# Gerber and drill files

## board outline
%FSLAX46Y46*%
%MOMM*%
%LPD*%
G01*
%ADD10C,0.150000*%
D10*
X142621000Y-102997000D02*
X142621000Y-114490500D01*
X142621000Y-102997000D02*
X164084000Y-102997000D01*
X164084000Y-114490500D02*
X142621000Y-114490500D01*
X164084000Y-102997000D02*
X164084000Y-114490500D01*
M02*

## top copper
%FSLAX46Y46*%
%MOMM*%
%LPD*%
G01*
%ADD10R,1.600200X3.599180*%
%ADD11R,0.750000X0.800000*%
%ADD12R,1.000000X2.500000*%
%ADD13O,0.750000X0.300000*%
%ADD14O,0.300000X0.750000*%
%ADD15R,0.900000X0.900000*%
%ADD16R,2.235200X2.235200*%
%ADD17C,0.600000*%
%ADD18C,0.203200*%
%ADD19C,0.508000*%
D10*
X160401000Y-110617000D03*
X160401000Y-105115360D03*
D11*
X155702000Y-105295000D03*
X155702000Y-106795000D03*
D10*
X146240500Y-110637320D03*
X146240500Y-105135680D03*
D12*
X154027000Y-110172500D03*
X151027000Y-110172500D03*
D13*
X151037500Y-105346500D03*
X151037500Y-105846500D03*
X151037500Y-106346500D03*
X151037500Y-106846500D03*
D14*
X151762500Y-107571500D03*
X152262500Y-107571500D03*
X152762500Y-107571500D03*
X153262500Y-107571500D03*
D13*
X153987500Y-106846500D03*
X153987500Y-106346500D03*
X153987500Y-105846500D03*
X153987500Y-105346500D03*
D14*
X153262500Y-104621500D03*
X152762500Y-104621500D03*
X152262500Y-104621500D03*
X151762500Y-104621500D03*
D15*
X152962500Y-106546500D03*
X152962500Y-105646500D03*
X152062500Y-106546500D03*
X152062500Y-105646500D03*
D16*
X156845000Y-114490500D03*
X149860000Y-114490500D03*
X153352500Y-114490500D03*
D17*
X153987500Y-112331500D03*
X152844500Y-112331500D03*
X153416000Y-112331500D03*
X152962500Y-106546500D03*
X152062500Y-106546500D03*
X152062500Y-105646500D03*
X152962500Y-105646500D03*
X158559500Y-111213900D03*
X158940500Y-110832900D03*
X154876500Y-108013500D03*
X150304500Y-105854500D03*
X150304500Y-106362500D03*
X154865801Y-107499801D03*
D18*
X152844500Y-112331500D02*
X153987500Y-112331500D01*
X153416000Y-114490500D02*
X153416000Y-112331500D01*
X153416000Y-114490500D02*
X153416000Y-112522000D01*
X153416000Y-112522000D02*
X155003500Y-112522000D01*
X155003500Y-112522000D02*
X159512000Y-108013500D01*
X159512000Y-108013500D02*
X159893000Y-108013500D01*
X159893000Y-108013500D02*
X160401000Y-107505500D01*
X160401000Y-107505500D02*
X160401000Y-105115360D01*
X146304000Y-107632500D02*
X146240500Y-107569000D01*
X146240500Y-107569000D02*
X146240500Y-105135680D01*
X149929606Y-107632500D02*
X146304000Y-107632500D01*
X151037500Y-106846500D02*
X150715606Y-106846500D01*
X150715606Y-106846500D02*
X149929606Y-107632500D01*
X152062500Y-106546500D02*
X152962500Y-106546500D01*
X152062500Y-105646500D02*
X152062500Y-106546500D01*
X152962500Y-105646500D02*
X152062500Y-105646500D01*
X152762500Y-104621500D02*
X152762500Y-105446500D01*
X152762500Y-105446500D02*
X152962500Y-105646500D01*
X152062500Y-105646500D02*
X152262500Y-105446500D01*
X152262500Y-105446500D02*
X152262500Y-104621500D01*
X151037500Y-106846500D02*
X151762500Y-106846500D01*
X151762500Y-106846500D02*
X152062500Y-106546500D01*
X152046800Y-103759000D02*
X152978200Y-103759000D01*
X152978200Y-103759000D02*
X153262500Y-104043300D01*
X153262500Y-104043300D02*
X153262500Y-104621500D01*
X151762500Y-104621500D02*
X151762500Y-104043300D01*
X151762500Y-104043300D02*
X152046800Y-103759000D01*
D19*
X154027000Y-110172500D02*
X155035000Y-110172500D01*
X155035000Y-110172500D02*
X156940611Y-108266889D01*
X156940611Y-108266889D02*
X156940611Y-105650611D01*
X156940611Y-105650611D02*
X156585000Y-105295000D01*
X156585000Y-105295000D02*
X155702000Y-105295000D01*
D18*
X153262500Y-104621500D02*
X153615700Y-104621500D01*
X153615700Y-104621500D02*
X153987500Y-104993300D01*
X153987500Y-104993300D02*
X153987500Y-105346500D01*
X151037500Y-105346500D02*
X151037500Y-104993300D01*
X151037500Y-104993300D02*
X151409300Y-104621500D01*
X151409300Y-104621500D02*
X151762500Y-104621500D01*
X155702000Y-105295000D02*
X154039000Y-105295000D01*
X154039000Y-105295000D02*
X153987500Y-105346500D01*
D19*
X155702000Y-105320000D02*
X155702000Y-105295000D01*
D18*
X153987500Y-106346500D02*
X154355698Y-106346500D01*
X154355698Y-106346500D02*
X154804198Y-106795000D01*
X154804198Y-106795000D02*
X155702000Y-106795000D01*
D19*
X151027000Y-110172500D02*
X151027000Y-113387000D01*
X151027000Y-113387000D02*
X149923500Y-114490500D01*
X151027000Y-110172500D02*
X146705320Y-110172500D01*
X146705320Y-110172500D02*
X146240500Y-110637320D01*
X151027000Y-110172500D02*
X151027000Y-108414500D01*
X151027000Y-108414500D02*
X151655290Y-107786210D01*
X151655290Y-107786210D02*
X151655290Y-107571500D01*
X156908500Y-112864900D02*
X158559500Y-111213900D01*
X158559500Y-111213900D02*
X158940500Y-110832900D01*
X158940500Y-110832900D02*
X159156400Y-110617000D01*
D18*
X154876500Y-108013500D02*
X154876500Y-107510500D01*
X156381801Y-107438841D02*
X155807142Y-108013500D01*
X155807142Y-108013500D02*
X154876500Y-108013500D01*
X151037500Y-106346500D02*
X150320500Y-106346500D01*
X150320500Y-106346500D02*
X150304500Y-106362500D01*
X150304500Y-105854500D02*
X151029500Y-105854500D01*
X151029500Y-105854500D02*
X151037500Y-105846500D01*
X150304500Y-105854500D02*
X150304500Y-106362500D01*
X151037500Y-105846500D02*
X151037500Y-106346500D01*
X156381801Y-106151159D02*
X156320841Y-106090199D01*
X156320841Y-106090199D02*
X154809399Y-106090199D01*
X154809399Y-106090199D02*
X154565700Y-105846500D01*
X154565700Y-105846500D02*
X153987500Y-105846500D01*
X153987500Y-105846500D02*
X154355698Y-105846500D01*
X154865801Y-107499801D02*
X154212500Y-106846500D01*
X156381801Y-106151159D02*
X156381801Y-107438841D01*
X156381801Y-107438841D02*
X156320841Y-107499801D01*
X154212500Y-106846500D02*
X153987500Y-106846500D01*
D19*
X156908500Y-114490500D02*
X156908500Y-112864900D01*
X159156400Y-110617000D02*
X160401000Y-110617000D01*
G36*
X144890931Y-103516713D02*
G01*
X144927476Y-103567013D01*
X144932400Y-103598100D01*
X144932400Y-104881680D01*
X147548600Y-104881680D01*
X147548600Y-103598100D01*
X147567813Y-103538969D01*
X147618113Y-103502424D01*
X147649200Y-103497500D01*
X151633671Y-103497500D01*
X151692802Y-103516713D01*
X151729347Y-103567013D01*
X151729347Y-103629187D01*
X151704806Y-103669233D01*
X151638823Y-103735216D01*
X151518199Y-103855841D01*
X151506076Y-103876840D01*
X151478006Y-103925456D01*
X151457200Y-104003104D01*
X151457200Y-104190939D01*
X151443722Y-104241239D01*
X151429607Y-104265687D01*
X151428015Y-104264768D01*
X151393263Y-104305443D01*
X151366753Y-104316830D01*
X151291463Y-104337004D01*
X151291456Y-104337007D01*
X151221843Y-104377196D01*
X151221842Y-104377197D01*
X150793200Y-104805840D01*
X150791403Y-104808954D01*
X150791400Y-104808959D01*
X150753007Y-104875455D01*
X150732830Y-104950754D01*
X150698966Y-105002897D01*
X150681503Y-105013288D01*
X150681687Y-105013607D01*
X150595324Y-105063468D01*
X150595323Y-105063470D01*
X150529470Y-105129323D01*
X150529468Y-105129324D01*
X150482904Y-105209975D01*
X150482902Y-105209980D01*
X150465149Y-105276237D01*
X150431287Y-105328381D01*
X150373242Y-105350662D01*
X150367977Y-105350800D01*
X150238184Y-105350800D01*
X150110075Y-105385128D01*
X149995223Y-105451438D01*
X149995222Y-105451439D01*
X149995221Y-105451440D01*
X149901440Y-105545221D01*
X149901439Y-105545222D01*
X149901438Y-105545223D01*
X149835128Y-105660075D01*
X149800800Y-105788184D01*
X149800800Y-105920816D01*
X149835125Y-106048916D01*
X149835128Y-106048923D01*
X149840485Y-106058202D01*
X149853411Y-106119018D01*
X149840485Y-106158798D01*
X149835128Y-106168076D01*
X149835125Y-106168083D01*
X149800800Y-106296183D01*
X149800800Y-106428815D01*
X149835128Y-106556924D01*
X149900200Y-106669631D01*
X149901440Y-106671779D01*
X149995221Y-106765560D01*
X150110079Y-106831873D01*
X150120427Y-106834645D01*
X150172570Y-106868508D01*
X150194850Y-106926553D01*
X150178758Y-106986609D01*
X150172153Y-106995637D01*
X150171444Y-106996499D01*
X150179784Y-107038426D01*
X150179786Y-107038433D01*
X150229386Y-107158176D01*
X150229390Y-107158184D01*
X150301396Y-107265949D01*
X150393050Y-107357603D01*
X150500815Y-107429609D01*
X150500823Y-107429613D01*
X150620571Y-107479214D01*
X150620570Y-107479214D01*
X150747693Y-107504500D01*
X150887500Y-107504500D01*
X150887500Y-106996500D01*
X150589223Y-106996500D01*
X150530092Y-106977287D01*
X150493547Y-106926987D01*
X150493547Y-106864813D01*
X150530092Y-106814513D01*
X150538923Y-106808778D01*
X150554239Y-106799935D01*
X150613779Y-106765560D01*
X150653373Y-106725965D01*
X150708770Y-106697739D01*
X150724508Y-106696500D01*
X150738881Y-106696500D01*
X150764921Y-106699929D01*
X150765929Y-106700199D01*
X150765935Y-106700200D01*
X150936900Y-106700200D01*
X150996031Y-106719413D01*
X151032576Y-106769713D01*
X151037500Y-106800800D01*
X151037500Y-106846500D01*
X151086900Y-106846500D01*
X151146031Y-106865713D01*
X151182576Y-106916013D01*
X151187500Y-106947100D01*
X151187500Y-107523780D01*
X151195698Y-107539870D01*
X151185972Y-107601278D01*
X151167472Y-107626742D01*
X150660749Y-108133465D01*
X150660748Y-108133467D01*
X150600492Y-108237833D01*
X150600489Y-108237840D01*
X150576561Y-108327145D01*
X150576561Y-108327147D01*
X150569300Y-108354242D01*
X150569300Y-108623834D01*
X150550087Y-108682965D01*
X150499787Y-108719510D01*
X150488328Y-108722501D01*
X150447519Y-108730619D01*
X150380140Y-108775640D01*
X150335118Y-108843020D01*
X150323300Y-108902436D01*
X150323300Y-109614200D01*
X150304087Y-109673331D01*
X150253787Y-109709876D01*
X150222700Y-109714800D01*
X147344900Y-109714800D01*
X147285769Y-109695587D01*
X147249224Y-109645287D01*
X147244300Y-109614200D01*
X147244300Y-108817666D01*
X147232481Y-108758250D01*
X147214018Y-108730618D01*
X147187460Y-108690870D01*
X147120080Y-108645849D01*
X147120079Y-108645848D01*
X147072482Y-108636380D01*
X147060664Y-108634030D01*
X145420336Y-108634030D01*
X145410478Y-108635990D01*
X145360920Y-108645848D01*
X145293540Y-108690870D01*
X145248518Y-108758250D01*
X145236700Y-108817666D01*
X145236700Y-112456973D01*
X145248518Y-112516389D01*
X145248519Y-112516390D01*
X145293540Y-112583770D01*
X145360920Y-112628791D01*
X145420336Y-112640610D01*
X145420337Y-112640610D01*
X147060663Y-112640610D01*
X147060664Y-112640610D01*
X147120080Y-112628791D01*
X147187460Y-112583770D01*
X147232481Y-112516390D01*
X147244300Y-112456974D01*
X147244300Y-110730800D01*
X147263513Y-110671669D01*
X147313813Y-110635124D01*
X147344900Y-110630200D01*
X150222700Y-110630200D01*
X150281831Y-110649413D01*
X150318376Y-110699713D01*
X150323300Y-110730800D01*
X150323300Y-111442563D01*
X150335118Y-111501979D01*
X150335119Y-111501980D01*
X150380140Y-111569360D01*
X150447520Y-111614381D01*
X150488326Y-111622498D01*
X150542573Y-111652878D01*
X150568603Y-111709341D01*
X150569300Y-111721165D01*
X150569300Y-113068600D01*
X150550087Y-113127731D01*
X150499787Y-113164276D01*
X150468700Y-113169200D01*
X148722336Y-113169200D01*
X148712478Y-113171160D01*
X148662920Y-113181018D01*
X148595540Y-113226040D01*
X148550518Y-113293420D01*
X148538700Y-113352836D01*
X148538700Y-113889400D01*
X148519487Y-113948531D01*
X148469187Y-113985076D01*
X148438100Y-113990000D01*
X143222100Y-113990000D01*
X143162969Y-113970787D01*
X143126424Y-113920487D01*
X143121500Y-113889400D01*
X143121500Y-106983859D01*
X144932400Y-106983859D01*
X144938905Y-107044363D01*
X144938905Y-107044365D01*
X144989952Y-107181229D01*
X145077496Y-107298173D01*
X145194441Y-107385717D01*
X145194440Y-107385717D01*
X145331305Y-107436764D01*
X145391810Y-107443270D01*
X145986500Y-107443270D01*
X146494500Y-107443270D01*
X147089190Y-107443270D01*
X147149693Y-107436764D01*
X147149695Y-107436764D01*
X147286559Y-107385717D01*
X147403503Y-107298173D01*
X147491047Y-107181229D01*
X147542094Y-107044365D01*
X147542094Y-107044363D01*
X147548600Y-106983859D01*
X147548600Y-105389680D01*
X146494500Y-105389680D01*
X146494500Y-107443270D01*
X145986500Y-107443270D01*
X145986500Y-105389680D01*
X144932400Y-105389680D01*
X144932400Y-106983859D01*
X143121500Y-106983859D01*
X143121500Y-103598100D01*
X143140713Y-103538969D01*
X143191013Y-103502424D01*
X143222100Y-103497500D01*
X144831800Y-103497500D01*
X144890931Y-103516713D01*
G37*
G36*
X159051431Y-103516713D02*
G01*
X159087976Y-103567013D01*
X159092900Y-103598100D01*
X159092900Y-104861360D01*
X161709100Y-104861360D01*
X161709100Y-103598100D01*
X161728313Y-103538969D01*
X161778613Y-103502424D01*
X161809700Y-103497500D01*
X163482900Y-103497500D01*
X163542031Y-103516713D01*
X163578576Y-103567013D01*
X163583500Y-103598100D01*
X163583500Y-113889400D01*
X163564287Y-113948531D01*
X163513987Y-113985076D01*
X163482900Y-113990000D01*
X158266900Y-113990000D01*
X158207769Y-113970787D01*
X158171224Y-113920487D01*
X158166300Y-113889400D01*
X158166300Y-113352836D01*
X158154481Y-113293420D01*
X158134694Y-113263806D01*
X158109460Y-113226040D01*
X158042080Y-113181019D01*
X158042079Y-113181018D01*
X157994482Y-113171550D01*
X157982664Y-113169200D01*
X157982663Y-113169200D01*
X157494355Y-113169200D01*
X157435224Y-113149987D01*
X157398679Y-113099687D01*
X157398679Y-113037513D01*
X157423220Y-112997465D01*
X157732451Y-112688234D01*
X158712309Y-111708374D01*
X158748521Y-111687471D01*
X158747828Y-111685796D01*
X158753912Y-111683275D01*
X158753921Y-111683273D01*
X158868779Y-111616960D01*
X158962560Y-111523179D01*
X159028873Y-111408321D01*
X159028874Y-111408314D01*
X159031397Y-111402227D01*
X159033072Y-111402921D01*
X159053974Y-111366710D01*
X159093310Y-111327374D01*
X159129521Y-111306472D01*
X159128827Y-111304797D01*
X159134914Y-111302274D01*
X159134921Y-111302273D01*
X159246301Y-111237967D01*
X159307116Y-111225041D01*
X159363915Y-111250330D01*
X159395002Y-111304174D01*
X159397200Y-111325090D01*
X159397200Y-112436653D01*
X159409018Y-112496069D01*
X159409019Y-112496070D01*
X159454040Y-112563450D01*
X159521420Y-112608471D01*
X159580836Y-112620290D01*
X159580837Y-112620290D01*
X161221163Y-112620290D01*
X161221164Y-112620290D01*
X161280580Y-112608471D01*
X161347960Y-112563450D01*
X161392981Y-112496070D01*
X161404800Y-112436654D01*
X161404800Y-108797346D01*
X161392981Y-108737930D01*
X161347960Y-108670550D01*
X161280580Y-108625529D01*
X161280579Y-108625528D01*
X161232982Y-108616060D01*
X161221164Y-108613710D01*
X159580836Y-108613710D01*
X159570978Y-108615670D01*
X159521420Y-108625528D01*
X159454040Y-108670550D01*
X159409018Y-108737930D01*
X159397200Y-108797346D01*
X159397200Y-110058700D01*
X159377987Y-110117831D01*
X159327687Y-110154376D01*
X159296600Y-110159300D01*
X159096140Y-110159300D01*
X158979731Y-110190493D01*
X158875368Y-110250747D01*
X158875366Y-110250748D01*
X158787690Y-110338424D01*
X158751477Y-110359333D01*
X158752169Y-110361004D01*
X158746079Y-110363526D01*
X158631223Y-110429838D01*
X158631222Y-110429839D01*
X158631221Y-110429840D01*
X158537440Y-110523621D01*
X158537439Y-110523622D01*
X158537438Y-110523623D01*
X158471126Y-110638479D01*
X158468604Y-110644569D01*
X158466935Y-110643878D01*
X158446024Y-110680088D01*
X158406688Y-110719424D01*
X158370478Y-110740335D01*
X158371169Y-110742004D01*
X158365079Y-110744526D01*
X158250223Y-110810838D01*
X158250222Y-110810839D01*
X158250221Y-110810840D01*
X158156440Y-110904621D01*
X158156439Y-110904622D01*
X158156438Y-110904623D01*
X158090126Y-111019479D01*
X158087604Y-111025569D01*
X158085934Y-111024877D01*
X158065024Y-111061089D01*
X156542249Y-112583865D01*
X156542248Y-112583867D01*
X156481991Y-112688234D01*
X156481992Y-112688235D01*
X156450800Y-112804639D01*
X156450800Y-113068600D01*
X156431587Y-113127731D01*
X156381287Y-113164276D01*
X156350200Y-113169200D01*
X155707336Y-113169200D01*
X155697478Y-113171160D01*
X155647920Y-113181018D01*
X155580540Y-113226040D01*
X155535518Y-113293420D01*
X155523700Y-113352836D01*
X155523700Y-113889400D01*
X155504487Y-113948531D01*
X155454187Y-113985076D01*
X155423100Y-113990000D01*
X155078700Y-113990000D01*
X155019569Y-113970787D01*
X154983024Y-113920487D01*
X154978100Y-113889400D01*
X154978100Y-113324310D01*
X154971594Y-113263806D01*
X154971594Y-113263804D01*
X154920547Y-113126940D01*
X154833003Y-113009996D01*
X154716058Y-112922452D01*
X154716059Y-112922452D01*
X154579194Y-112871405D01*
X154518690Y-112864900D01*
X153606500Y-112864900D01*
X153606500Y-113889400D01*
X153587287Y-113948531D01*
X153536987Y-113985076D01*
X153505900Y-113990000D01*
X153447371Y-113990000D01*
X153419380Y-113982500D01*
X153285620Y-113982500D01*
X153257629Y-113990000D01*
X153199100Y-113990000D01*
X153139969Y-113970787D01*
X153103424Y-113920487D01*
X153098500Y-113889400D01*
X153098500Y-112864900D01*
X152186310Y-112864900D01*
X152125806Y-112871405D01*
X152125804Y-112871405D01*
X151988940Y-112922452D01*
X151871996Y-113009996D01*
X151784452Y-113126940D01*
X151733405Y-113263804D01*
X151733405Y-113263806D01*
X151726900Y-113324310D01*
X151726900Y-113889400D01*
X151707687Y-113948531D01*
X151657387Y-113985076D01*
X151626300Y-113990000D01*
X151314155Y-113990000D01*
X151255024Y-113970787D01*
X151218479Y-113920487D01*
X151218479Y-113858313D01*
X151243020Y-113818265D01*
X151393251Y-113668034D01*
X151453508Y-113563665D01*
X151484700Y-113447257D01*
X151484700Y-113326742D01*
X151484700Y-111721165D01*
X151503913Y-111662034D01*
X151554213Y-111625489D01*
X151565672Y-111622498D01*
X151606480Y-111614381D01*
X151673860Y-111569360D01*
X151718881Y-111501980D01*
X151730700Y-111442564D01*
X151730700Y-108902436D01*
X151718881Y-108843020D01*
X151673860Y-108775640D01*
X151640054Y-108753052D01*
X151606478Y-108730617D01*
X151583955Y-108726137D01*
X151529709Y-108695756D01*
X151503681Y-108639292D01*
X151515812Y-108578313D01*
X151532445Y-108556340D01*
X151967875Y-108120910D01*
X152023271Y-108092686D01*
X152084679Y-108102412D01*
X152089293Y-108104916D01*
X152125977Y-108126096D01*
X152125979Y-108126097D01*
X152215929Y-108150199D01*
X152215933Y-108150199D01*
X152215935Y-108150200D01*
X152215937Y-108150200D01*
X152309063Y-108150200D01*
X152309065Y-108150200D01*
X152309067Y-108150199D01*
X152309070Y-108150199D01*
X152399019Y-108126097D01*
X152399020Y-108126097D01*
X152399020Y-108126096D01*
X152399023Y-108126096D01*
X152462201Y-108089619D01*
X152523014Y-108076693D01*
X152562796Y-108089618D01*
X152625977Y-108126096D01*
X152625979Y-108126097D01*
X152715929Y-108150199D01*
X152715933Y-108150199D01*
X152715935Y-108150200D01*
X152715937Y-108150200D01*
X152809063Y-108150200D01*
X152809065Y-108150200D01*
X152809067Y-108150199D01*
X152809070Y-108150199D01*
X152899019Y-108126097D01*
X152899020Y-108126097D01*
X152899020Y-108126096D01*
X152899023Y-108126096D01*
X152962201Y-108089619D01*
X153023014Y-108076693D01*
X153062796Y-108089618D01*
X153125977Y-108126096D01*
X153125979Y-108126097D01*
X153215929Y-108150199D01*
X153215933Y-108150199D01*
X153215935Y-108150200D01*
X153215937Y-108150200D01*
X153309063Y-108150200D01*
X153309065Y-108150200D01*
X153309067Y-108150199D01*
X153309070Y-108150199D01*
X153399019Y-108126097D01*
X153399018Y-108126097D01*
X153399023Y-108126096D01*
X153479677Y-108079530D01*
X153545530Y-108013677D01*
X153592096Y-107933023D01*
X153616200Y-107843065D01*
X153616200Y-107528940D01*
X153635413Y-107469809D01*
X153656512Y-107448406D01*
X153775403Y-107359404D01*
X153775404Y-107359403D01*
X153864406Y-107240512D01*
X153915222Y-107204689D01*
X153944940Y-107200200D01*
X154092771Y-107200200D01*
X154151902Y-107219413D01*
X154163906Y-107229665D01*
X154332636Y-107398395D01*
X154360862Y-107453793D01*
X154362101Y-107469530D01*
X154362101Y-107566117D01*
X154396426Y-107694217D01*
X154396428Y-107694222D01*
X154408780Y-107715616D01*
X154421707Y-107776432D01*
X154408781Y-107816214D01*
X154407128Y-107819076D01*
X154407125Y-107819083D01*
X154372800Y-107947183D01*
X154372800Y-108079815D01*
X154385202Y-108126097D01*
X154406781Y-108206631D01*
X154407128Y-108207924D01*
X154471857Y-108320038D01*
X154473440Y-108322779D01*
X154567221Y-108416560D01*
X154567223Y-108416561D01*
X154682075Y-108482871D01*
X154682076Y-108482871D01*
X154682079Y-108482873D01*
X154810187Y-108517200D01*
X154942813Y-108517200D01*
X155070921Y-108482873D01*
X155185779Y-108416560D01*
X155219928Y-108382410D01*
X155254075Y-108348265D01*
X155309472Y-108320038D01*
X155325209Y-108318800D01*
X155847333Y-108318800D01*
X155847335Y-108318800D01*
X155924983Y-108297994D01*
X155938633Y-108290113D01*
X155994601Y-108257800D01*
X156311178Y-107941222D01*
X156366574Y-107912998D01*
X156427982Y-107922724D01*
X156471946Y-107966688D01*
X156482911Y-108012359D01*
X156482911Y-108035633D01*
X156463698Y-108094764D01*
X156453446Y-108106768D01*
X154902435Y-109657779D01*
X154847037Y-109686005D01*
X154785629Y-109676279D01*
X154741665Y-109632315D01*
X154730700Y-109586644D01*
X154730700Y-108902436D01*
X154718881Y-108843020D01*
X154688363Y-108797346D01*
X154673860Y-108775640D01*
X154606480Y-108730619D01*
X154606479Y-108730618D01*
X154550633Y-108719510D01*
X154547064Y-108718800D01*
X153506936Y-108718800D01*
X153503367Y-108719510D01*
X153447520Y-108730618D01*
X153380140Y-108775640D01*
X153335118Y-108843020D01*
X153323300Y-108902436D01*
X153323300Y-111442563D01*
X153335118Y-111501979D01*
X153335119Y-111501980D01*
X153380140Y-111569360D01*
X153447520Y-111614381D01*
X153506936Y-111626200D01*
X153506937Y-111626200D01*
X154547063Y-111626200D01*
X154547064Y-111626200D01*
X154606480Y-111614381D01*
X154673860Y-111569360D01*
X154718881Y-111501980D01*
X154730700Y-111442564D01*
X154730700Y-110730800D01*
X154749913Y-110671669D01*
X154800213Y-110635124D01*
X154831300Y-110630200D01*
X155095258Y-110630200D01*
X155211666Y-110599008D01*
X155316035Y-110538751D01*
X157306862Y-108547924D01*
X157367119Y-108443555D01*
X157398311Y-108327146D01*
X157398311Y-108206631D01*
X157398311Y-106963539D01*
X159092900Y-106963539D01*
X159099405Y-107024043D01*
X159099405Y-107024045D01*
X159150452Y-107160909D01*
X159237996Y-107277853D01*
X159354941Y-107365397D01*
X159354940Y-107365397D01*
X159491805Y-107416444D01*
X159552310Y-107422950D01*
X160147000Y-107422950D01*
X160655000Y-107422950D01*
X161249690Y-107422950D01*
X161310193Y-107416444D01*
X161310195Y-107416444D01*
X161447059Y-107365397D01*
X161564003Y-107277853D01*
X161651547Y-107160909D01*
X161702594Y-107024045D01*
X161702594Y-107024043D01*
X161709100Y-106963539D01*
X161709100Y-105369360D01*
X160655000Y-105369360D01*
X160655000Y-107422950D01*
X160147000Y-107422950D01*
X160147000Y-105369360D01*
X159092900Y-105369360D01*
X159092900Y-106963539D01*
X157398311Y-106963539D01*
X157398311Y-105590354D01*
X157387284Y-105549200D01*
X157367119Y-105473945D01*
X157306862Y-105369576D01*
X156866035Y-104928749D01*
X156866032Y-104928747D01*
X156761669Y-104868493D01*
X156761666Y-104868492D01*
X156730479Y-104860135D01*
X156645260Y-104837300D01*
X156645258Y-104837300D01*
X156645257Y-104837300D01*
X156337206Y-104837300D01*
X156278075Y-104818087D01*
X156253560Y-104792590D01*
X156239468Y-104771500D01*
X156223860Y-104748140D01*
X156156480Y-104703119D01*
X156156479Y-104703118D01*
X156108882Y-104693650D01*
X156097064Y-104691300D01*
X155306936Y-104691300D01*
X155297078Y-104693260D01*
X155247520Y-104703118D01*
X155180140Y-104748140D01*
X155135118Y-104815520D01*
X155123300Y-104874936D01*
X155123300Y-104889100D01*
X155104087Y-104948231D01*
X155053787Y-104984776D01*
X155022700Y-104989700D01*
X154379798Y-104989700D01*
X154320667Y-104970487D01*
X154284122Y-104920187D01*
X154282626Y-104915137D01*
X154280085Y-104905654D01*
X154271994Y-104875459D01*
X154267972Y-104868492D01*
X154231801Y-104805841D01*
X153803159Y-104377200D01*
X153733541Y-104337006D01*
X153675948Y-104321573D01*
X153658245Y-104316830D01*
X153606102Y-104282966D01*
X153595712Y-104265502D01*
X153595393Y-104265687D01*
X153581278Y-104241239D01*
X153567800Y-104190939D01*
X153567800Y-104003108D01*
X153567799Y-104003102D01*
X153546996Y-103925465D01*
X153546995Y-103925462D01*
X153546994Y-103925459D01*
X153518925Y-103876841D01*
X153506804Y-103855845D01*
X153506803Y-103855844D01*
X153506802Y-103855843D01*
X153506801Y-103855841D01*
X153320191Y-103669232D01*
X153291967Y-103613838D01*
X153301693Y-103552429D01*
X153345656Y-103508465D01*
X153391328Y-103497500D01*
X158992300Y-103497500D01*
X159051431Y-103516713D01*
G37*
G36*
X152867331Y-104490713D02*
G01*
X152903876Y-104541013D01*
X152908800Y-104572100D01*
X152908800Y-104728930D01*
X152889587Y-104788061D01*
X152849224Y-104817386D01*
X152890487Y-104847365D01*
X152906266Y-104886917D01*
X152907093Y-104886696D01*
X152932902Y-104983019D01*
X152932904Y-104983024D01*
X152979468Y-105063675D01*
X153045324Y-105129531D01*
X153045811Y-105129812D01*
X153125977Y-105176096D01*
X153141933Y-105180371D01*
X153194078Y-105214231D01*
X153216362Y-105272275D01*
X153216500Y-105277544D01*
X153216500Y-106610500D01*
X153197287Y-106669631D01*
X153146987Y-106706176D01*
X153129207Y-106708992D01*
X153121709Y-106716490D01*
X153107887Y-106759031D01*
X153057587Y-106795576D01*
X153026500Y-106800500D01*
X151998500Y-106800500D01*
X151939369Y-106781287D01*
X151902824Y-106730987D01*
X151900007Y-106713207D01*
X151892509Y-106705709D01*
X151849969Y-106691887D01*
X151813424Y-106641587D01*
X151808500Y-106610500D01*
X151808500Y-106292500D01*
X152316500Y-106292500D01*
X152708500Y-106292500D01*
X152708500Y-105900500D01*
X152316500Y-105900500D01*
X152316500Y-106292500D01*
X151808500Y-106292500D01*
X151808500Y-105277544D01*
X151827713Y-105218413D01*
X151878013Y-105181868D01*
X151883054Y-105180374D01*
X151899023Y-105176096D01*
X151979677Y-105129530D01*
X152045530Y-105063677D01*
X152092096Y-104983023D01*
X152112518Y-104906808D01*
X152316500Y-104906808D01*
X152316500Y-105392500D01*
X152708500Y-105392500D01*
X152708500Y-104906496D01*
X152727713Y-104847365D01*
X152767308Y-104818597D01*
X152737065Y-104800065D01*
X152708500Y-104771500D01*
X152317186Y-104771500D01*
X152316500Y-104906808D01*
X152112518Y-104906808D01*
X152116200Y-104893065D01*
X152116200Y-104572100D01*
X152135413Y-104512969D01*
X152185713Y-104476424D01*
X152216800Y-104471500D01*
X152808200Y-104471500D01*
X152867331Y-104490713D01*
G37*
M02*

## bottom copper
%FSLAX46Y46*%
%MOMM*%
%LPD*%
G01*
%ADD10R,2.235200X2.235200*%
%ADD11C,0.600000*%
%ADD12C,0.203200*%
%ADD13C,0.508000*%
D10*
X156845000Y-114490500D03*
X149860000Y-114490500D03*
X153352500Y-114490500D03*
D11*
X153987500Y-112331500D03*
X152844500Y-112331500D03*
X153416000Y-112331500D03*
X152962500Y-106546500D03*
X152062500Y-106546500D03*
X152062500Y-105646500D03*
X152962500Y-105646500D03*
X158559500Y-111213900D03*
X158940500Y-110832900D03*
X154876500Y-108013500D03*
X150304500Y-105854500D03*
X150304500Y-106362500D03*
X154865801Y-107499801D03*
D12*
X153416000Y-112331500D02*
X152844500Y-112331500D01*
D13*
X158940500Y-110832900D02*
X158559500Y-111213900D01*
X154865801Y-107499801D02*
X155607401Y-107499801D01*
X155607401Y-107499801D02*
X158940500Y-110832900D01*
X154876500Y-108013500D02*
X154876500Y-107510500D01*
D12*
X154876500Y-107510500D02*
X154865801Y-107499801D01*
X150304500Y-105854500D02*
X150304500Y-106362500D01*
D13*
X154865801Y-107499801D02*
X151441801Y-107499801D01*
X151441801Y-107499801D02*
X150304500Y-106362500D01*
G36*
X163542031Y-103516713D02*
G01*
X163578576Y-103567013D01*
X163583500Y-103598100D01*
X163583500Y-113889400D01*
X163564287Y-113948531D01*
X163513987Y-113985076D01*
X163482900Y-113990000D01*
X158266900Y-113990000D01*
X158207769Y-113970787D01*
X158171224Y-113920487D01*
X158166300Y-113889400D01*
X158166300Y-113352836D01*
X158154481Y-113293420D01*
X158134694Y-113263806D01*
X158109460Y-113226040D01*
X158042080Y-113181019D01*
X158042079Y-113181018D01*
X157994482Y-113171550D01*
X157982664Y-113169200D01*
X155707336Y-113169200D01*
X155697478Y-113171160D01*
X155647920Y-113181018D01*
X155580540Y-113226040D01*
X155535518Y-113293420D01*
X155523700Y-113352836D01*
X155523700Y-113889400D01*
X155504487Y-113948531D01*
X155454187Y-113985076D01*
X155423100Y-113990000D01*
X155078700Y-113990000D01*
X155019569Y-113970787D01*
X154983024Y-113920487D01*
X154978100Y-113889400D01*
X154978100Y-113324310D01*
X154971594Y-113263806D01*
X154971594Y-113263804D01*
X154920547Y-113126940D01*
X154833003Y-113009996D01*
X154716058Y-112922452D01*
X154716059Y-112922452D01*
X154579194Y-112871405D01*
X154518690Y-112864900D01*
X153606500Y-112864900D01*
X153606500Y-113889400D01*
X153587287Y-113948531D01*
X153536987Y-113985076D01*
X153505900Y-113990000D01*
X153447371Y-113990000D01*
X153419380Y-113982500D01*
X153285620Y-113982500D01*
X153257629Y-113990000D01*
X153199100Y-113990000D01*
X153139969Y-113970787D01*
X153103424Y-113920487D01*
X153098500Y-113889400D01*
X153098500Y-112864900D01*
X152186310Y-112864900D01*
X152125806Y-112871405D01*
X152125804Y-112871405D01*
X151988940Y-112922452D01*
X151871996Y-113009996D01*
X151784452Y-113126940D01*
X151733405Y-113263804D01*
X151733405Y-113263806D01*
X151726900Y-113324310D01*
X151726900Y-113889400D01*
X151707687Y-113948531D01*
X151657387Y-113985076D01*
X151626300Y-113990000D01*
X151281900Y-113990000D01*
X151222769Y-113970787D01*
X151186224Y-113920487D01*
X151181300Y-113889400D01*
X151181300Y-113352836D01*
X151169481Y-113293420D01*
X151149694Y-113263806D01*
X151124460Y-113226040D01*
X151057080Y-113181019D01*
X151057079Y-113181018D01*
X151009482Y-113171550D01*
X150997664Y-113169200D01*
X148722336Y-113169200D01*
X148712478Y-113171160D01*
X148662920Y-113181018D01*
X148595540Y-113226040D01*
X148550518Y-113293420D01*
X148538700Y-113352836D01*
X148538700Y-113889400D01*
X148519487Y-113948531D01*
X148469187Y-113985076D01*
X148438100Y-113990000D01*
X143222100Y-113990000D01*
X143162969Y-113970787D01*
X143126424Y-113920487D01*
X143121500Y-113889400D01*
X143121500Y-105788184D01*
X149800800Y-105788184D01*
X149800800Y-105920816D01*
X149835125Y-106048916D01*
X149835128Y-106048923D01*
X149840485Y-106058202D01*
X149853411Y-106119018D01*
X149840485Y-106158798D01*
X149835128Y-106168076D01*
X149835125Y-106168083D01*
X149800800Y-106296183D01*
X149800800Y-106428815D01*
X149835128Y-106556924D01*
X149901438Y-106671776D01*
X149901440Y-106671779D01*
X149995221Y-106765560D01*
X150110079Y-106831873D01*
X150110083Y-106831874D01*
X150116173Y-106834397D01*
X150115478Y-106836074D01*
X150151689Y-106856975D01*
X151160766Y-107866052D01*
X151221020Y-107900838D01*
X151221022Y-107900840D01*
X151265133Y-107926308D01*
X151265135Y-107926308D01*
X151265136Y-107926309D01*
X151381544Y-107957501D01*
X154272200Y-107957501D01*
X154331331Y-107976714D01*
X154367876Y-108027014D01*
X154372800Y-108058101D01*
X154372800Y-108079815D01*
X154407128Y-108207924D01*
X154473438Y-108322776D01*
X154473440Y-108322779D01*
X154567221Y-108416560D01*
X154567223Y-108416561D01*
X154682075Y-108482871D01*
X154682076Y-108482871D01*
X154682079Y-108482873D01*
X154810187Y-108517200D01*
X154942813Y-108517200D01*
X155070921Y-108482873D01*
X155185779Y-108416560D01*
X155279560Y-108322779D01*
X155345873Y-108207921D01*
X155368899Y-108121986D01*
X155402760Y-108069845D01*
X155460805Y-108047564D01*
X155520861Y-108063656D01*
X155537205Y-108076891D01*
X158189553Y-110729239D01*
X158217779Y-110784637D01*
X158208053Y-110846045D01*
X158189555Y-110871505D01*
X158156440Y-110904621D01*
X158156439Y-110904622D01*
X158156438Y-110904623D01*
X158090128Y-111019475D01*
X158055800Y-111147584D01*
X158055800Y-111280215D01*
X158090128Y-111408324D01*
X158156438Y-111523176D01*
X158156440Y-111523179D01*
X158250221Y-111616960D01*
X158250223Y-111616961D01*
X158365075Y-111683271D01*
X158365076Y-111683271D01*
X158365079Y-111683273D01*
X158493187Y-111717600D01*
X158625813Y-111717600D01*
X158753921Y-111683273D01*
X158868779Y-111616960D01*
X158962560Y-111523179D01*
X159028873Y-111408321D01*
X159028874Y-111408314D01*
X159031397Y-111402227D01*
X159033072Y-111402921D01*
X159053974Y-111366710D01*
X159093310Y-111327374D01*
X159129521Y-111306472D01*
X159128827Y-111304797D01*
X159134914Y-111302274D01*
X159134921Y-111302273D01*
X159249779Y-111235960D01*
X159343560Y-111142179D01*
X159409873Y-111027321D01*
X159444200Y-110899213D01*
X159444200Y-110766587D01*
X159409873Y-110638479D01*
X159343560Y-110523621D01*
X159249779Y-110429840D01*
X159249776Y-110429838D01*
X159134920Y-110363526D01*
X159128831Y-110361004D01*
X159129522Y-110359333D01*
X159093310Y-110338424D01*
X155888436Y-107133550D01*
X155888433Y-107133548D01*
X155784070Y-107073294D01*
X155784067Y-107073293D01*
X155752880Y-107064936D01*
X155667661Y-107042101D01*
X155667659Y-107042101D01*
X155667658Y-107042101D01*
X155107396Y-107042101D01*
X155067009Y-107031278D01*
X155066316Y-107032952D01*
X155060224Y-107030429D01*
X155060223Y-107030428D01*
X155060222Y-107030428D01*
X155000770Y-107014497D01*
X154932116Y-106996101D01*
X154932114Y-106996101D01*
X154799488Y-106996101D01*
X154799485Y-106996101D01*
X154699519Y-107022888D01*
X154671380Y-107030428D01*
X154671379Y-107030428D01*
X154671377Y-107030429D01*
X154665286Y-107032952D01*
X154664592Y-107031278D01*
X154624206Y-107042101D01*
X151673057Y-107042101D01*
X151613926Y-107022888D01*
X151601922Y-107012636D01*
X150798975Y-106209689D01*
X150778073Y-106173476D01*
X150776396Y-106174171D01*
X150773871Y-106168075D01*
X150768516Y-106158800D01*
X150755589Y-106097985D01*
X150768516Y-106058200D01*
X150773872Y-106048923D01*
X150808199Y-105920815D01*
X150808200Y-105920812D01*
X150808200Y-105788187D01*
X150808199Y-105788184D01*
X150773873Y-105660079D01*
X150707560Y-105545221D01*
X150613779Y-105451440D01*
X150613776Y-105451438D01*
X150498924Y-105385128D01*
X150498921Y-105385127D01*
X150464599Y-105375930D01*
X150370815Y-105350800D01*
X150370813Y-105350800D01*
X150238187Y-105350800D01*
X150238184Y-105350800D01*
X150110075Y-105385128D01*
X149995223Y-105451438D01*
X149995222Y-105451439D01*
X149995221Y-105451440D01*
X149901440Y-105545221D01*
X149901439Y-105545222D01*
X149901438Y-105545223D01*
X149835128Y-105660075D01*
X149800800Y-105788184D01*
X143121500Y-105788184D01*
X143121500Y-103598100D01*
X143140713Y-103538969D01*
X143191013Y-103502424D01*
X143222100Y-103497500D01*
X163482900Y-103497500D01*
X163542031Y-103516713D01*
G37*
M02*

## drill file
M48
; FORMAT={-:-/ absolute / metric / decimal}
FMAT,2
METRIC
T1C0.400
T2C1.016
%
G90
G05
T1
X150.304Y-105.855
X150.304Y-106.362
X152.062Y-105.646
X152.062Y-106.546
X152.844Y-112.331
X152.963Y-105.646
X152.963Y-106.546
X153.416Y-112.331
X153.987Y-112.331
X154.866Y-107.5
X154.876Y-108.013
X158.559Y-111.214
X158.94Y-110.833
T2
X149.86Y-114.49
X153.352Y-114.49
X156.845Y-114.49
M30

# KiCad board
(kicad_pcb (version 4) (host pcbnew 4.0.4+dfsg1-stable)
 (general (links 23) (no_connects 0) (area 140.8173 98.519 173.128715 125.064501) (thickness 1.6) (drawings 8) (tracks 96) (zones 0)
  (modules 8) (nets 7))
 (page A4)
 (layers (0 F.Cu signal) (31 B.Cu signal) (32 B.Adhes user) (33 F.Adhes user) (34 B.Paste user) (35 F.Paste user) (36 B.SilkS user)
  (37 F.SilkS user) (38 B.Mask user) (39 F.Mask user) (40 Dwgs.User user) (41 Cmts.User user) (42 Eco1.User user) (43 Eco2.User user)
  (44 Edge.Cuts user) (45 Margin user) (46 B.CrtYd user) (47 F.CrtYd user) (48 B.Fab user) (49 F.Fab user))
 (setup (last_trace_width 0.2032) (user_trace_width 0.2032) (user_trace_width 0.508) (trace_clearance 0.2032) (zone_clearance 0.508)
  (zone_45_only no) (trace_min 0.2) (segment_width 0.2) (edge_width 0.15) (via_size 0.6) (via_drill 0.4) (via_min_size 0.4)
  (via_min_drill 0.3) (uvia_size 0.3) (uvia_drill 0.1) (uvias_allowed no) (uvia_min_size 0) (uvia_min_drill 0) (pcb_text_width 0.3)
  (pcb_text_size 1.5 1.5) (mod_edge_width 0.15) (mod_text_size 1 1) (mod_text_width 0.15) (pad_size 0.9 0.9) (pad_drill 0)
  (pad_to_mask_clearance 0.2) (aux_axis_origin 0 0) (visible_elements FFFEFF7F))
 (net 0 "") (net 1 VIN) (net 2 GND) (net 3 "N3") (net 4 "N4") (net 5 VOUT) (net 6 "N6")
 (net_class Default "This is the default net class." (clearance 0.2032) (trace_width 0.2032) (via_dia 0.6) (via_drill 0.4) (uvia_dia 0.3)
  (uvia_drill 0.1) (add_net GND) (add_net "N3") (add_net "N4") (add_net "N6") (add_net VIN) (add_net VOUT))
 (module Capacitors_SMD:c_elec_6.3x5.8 (layer F.Cu) (at 160.401 107.86618 270)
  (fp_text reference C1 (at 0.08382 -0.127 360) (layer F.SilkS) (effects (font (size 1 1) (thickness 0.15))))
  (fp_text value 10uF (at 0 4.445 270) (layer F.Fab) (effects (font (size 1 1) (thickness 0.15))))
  (pad 1 smd rect (at 2.75082 0 270) (size 3.59918 1.6002) (layers F.Cu F.Paste F.Mask) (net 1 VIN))
  (pad 2 smd rect (at -2.75082 0 270) (size 3.59918 1.6002) (layers F.Cu F.Paste F.Mask) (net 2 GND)))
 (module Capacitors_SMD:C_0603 (layer F.Cu) (at 155.702 106.045 270)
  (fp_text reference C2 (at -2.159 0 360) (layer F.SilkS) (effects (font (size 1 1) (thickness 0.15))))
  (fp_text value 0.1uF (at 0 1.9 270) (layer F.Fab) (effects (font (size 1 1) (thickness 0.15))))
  (pad 1 smd rect (at -0.75 0 270) (size 0.8 0.75) (layers F.Cu F.Paste F.Mask) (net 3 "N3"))
  (pad 2 smd rect (at 0.75 0 270) (size 0.8 0.75) (layers F.Cu F.Paste F.Mask) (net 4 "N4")))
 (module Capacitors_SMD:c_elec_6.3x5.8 (layer F.Cu) (at 146.2405 107.8865 270)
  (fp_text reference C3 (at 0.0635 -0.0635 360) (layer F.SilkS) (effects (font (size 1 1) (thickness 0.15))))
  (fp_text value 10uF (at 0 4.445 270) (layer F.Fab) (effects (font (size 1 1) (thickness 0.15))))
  (pad 1 smd rect (at 2.75082 0 270) (size 3.59918 1.6002) (layers F.Cu F.Paste F.Mask) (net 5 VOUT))
  (pad 2 smd rect (at -2.75082 0 270) (size 3.59918 1.6002) (layers F.Cu F.Paste F.Mask) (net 2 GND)))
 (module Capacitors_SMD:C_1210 (layer F.Cu) (at 152.527 110.1725 180)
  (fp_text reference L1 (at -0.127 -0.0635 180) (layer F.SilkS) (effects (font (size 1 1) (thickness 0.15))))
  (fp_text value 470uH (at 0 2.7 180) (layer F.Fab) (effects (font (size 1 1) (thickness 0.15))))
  (pad 1 smd rect (at -1.5 0 180) (size 1 2.5) (layers F.Cu F.Paste F.Mask) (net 3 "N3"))
  (pad 2 smd rect (at 1.5 0 180) (size 1 2.5) (layers F.Cu F.Paste F.Mask) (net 5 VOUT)))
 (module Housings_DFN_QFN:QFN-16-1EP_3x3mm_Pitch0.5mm (layer F.Cu) (at 152.5125 106.0965)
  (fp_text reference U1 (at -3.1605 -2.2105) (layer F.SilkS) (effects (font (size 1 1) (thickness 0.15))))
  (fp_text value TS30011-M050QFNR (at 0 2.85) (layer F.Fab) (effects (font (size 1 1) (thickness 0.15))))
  (pad 1 smd oval (at -1.475 -0.75) (size 0.75 0.3) (layers F.Cu F.Paste F.Mask) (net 3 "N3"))
  (pad 2 smd oval (at -1.475 -0.25) (size 0.75 0.3) (layers F.Cu F.Paste F.Mask) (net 1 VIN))
  (pad 3 smd oval (at -1.475 0.25) (size 0.75 0.3) (layers F.Cu F.Paste F.Mask) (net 1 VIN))
  (pad 4 smd oval (at -1.475 0.75) (size 0.75 0.3) (layers F.Cu F.Paste F.Mask) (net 2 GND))
  (pad 5 smd oval (at -0.75 1.475 90) (size 0.75 0.3) (layers F.Cu F.Paste F.Mask) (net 5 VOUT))
  (pad 6 smd oval (at -0.25 1.475 90) (size 0.75 0.3) (layers F.Cu F.Paste F.Mask))
  (pad 7 smd oval (at 0.25 1.475 90) (size 0.75 0.3) (layers F.Cu F.Paste F.Mask))
  (pad 8 smd oval (at 0.75 1.475 90) (size 0.75 0.3) (layers F.Cu F.Paste F.Mask) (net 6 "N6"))
  (pad 9 smd oval (at 1.475 0.75) (size 0.75 0.3) (layers F.Cu F.Paste F.Mask) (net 1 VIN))
  (pad 10 smd oval (at 1.475 0.25) (size 0.75 0.3) (layers F.Cu F.Paste F.Mask) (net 4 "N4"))
  (pad 11 smd oval (at 1.475 -0.25) (size 0.75 0.3) (layers F.Cu F.Paste F.Mask) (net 1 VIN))
  (pad 12 smd oval (at 1.475 -0.75) (size 0.75 0.3) (layers F.Cu F.Paste F.Mask) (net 3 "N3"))
  (pad 13 smd oval (at 0.75 -1.475 90) (size 0.75 0.3) (layers F.Cu F.Paste F.Mask) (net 3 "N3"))
  (pad 14 smd oval (at 0.25 -1.475 90) (size 0.75 0.3) (layers F.Cu F.Paste F.Mask) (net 2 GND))
  (pad 15 smd oval (at -0.25 -1.475 90) (size 0.75 0.3) (layers F.Cu F.Paste F.Mask) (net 2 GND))
  (pad 16 smd oval (at -0.75 -1.475 90) (size 0.75 0.3) (layers F.Cu F.Paste F.Mask) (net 3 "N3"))
  (pad 17 smd rect (at 0.45 0.45) (size 0.9 0.9) (layers F.Cu F.Paste F.Mask) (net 2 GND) (solder_paste_margin_ratio -0.2))
  (pad 17 smd rect (at 0.45 -0.45) (size 0.9 0.9) (layers F.Cu F.Paste F.Mask) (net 2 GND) (solder_paste_margin_ratio -0.2))
  (pad 17 smd rect (at -0.45 0.45) (size 0.9 0.9) (layers F.Cu F.Paste F.Mask) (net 2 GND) (solder_paste_margin_ratio -0.2))
  (pad 17 smd rect (at -0.45 -0.45) (size 0.9 0.9) (layers F.Cu F.Paste F.Mask) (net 2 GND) (solder_paste_margin_ratio -0.2)))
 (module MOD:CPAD (layer F.Cu) (at 156.845 114.4905)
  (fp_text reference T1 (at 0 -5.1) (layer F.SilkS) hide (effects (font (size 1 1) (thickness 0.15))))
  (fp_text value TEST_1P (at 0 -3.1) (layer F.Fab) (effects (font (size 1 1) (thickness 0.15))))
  (pad 1 thru_hole rect (at 0 0) (size 2.2352 2.2352) (drill 1.016) (layers *.Cu *.Mask F.SilkS) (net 1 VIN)))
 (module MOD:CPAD (layer F.Cu) (at 149.86 114.4905)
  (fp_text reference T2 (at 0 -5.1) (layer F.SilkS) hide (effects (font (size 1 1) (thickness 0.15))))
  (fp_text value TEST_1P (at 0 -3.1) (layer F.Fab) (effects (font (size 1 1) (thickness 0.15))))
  (pad 1 thru_hole rect (at 0 0) (size 2.2352 2.2352) (drill 1.016) (layers *.Cu *.Mask F.SilkS) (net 5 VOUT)))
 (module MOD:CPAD (layer F.Cu) (at 153.3525 114.4905)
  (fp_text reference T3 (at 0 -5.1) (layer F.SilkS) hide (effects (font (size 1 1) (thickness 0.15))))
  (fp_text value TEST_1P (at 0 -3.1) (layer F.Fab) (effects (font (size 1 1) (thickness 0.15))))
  (pad 1 thru_hole rect (at 0 0) (size 2.2352 2.2352) (drill 1.016) (layers *.Cu *.Mask F.SilkS) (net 2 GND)))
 (gr_line (start 142.621 102.997) (end 142.621 114.4905) (layer Edge.Cuts) (width 0.15))
 (gr_line (start 142.621 102.997) (end 164.084 102.997) (layer Edge.Cuts) (width 0.15))
 (gr_line (start 164.084 114.4905) (end 142.621 114.4905) (layer Edge.Cuts) (width 0.15))
 (gr_line (start 164.084 102.997) (end 164.084 114.4905) (layer Edge.Cuts) (width 0.15))
 (segment (start 152.8445 112.3315) (end 153.9875 112.3315) (width 0.2032) (layer F.Cu) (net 2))
 (via (at 153.9875 112.3315) (size 0.6) (drill 0.4) (layers F.Cu B.Cu) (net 2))
 (segment (start 153.416 112.3315) (end 152.8445 112.3315) (width 0.2032) (layer B.Cu) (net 2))
 (via (at 152.8445 112.3315) (size 0.6) (drill 0.4) (layers F.Cu B.Cu) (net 2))
 (segment (start 153.416 114.4905) (end 153.416 112.3315) (width 0.2032) (layer F.Cu) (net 2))
 (via (at 153.416 112.3315) (size 0.6) (drill 0.4) (layers F.Cu B.Cu) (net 2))
 (segment (start 153.416 114.4905) (end 153.416 112.522) (width 0.2032) (layer F.Cu) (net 2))
 (segment (start 153.416 112.522) (end 155.0035 112.522) (width 0.2032) (layer F.Cu) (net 2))
 (segment (start 155.0035 112.522) (end 159.512 108.0135) (width 0.2032) (layer F.Cu) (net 2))
 (segment (start 159.512 108.0135) (end 159.893 108.0135) (width 0.2032) (layer F.Cu) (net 2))
 (segment (start 159.893 108.0135) (end 160.401 107.5055) (width 0.2032) (layer F.Cu) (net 2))
 (segment (start 160.401 107.5055) (end 160.401 105.11536) (width 0.2032) (layer F.Cu) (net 2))
 (segment (start 146.304 107.6325) (end 146.2405 107.569) (width 0.2032) (layer F.Cu) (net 2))
 (segment (start 146.2405 107.569) (end 146.2405 105.13568) (width 0.2032) (layer F.Cu) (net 2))
 (segment (start 149.929606 107.6325) (end 146.304 107.6325) (width 0.2032) (layer F.Cu) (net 2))
 (segment (start 151.0375 106.8465) (end 150.715606 106.8465) (width 0.2032) (layer F.Cu) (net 2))
 (segment (start 150.715606 106.8465) (end 149.929606 107.6325) (width 0.2032) (layer F.Cu) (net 2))
 (segment (start 152.0625 106.5465) (end 152.9625 106.5465) (width 0.2032) (layer F.Cu) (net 2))
 (via (at 152.9625 106.5465) (size 0.6) (drill 0.4) (layers F.Cu B.Cu) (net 2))
 (segment (start 152.0625 105.6465) (end 152.0625 106.5465) (width 0.2032) (layer F.Cu) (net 2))
 (via (at 152.0625 106.5465) (size 0.6) (drill 0.4) (layers F.Cu B.Cu) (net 2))
 (segment (start 152.9625 105.6465) (end 152.0625 105.6465) (width 0.2032) (layer F.Cu) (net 2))
 (via (at 152.0625 105.6465) (size 0.6) (drill 0.4) (layers F.Cu B.Cu) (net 2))
 (via (at 152.9625 105.6465) (size 0.6) (drill 0.4) (layers F.Cu B.Cu) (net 2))
 (segment (start 152.7625 104.6215) (end 152.7625 105.4465) (width 0.2032) (layer F.Cu) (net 2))
 (segment (start 152.7625 105.4465) (end 152.9625 105.6465) (width 0.2032) (layer F.Cu) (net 2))
 (segment (start 152.0625 105.6465) (end 152.2625 105.4465) (width 0.2032) (layer F.Cu) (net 2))
 (segment (start 152.2625 105.4465) (end 152.2625 104.6215) (width 0.2032) (layer F.Cu) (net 2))
 (segment (start 151.0375 106.8465) (end 151.7625 106.8465) (width 0.2032) (layer F.Cu) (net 2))
 (segment (start 151.7625 106.8465) (end 152.0625 106.5465) (width 0.2032) (layer F.Cu) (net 2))
 (segment (start 152.0468 103.759) (end 152.9782 103.759) (width 0.2032) (layer F.Cu) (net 3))
 (segment (start 152.9782 103.759) (end 153.2625 104.0433) (width 0.2032) (layer F.Cu) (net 3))
 (segment (start 153.2625 104.0433) (end 153.2625 104.6215) (width 0.2032) (layer F.Cu) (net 3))
 (segment (start 151.7625 104.6215) (end 151.7625 104.0433) (width 0.2032) (layer F.Cu) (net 3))
 (segment (start 151.7625 104.0433) (end 152.0468 103.759) (width 0.2032) (layer F.Cu) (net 3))
 (segment (start 154.027 110.1725) (end 155.035 110.1725) (width 0.508) (layer F.Cu) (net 3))
 (segment (start 155.035 110.1725) (end 156.940611 108.266889) (width 0.508) (layer F.Cu) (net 3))
 (segment (start 156.940611 108.266889) (end 156.940611 105.650611) (width 0.508) (layer F.Cu) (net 3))
 (segment (start 156.940611 105.650611) (end 156.585 105.295) (width 0.508) (layer F.Cu) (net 3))
 (segment (start 156.585 105.295) (end 155.702 105.295) (width 0.508) (layer F.Cu) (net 3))
 (segment (start 153.2625 104.6215) (end 153.6157 104.6215) (width 0.2032) (layer F.Cu) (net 3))
 (segment (start 153.6157 104.6215) (end 153.9875 104.9933) (width 0.2032) (layer F.Cu) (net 3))
 (segment (start 153.9875 104.9933) (end 153.9875 105.3465) (width 0.2032) (layer F.Cu) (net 3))
 (segment (start 151.0375 105.3465) (end 151.0375 104.9933) (width 0.2032) (layer F.Cu) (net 3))
 (segment (start 151.0375 104.9933) (end 151.4093 104.6215) (width 0.2032) (layer F.Cu) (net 3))
 (segment (start 151.4093 104.6215) (end 151.7625 104.6215) (width 0.2032) (layer F.Cu) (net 3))
 (segment (start 155.702 105.295) (end 154.039 105.295) (width 0.2032) (layer F.Cu) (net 3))
 (segment (start 154.039 105.295) (end 153.9875 105.3465) (width 0.2032) (layer F.Cu) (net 3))
 (segment (start 155.702 105.32) (end 155.702 105.295) (width 0.508) (layer F.Cu) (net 3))
 (segment (start 153.9875 106.3465) (end 154.355698 106.3465) (width 0.2032) (layer F.Cu) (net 4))
 (segment (start 154.355698 106.3465) (end 154.804198 106.795) (width 0.2032) (layer F.Cu) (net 4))
 (segment (start 154.804198 106.795) (end 155.702 106.795) (width 0.2032) (layer F.Cu) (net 4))
 (segment (start 151.027 110.1725) (end 151.027 113.387) (width 0.508) (layer F.Cu) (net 5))
 (segment (start 151.027 113.387) (end 149.9235 114.4905) (width 0.508) (layer F.Cu) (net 5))
 (segment (start 151.027 110.1725) (end 146.70532 110.1725) (width 0.508) (layer F.Cu) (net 5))
 (segment (start 146.70532 110.1725) (end 146.2405 110.63732) (width 0.508) (layer F.Cu) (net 5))
 (segment (start 151.027 110.1725) (end 151.027 108.4145) (width 0.508) (layer F.Cu) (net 5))
 (segment (start 151.027 108.4145) (end 151.65529 107.78621) (width 0.508) (layer F.Cu) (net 5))
 (segment (start 151.65529 107.78621) (end 151.65529 107.5715) (width 0.508) (layer F.Cu) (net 5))
 (segment (start 156.9085 112.8649) (end 158.5595 111.2139) (width 0.508) (layer F.Cu) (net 1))
 (segment (start 158.5595 111.2139) (end 158.9405 110.8329) (width 0.508) (layer F.Cu) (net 1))
 (segment (start 158.9405 110.8329) (end 158.5595 111.2139) (width 0.508) (layer B.Cu) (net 1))
 (via (at 158.5595 111.2139) (size 0.6) (drill 0.4) (layers F.Cu B.Cu) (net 1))
 (segment (start 158.9405 110.8329) (end 159.1564 110.617) (width 0.508) (layer F.Cu) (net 1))
 (segment (start 154.865801 107.499801) (end 155.607401 107.499801) (width 0.508) (layer B.Cu) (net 1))
 (via (at 158.9405 110.8329) (size 0.6) (drill 0.4) (layers F.Cu B.Cu) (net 1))
 (segment (start 155.607401 107.499801) (end 158.9405 110.8329) (width 0.508) (layer B.Cu) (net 1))
 (segment (start 154.8765 108.0135) (end 154.8765 107.5105) (width 0.2032) (layer F.Cu) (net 1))
 (segment (start 154.8765 108.0135) (end 154.8765 107.5105) (width 0.508) (layer B.Cu) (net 1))
 (segment (start 154.8765 107.5105) (end 154.865801 107.499801) (width 0.2032) (layer B.Cu) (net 1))
 (segment (start 156.381801 107.438841) (end 155.807142 108.0135) (width 0.2032) (layer F.Cu) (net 1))
 (segment (start 155.807142 108.0135) (end 154.8765 108.0135) (width 0.2032) (layer F.Cu) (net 1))
 (via (at 154.8765 108.0135) (size 0.6) (drill 0.4) (layers F.Cu B.Cu) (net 1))
 (segment (start 151.0375 106.3465) (end 150.3205 106.3465) (width 0.2032) (layer F.Cu) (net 1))
 (segment (start 150.3205 106.3465) (end 150.3045 106.3625) (width 0.2032) (layer F.Cu) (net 1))
 (segment (start 150.3045 105.8545) (end 151.0295 105.8545) (width 0.2032) (layer F.Cu) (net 1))
 (segment (start 151.0295 105.8545) (end 151.0375 105.8465) (width 0.2032) (layer F.Cu) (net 1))
 (segment (start 150.3045 105.8545) (end 150.3045 106.3625) (width 0.2032) (layer F.Cu) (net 1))
 (segment (start 150.3045 105.8545) (end 150.3045 106.3625) (width 0.2032) (layer B.Cu) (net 1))
 (via (at 150.3045 105.8545) (size 0.6) (drill 0.4) (layers F.Cu B.Cu) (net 1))
 (segment (start 154.865801 107.499801) (end 151.441801 107.499801) (width 0.508) (layer B.Cu) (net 1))
 (segment (start 151.441801 107.499801) (end 150.3045 106.3625) (width 0.508) (layer B.Cu) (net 1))
 (via (at 150.3045 106.3625) (size 0.6) (drill 0.4) (layers F.Cu B.Cu) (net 1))
 (via (at 154.865801 107.499801) (size 0.6) (drill 0.4) (layers F.Cu B.Cu) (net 1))
 (segment (start 151.0375 105.8465) (end 151.0375 106.3465) (width 0.2032) (layer F.Cu) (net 1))
 (segment (start 156.381801 106.151159) (end 156.320841 106.090199) (width 0.2032) (layer F.Cu) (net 1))
 (segment (start 156.320841 106.090199) (end 154.809399 106.090199) (width 0.2032) (layer F.Cu) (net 1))
 (segment (start 154.809399 106.090199) (end 154.5657 105.8465) (width 0.2032) (layer F.Cu) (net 1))
 (segment (start 154.5657 105.8465) (end 153.9875 105.8465) (width 0.2032) (layer F.Cu) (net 1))
 (segment (start 153.9875 105.8465) (end 154.355698 105.8465) (width 0.2032) (layer F.Cu) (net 1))
 (segment (start 154.865801 107.499801) (end 154.2125 106.8465) (width 0.2032) (layer F.Cu) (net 1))
 (segment (start 156.381801 106.151159) (end 156.381801 107.438841) (width 0.2032) (layer F.Cu) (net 1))
 (segment (start 156.381801 107.438841) (end 156.320841 107.499801) (width 0.2032) (layer F.Cu) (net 1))
 (segment (start 154.2125 106.8465) (end 153.9875 106.8465) (width 0.2032) (layer F.Cu) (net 1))
 (segment (start 156.9085 114.4905) (end 156.9085 112.8649) (width 0.508) (layer F.Cu) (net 1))
 (segment (start 159.1564 110.617) (end 160.401 110.617) (width 0.508) (layer F.Cu) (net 1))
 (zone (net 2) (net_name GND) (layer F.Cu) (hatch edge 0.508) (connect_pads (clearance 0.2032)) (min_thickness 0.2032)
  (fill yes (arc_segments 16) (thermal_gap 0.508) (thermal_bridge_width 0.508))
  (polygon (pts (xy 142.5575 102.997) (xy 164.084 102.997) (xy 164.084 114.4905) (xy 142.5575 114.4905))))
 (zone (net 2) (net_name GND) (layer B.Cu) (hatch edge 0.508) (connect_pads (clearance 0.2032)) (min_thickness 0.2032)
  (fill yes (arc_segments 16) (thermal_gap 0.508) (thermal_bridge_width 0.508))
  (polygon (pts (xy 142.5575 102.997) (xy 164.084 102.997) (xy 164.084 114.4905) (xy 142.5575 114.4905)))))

